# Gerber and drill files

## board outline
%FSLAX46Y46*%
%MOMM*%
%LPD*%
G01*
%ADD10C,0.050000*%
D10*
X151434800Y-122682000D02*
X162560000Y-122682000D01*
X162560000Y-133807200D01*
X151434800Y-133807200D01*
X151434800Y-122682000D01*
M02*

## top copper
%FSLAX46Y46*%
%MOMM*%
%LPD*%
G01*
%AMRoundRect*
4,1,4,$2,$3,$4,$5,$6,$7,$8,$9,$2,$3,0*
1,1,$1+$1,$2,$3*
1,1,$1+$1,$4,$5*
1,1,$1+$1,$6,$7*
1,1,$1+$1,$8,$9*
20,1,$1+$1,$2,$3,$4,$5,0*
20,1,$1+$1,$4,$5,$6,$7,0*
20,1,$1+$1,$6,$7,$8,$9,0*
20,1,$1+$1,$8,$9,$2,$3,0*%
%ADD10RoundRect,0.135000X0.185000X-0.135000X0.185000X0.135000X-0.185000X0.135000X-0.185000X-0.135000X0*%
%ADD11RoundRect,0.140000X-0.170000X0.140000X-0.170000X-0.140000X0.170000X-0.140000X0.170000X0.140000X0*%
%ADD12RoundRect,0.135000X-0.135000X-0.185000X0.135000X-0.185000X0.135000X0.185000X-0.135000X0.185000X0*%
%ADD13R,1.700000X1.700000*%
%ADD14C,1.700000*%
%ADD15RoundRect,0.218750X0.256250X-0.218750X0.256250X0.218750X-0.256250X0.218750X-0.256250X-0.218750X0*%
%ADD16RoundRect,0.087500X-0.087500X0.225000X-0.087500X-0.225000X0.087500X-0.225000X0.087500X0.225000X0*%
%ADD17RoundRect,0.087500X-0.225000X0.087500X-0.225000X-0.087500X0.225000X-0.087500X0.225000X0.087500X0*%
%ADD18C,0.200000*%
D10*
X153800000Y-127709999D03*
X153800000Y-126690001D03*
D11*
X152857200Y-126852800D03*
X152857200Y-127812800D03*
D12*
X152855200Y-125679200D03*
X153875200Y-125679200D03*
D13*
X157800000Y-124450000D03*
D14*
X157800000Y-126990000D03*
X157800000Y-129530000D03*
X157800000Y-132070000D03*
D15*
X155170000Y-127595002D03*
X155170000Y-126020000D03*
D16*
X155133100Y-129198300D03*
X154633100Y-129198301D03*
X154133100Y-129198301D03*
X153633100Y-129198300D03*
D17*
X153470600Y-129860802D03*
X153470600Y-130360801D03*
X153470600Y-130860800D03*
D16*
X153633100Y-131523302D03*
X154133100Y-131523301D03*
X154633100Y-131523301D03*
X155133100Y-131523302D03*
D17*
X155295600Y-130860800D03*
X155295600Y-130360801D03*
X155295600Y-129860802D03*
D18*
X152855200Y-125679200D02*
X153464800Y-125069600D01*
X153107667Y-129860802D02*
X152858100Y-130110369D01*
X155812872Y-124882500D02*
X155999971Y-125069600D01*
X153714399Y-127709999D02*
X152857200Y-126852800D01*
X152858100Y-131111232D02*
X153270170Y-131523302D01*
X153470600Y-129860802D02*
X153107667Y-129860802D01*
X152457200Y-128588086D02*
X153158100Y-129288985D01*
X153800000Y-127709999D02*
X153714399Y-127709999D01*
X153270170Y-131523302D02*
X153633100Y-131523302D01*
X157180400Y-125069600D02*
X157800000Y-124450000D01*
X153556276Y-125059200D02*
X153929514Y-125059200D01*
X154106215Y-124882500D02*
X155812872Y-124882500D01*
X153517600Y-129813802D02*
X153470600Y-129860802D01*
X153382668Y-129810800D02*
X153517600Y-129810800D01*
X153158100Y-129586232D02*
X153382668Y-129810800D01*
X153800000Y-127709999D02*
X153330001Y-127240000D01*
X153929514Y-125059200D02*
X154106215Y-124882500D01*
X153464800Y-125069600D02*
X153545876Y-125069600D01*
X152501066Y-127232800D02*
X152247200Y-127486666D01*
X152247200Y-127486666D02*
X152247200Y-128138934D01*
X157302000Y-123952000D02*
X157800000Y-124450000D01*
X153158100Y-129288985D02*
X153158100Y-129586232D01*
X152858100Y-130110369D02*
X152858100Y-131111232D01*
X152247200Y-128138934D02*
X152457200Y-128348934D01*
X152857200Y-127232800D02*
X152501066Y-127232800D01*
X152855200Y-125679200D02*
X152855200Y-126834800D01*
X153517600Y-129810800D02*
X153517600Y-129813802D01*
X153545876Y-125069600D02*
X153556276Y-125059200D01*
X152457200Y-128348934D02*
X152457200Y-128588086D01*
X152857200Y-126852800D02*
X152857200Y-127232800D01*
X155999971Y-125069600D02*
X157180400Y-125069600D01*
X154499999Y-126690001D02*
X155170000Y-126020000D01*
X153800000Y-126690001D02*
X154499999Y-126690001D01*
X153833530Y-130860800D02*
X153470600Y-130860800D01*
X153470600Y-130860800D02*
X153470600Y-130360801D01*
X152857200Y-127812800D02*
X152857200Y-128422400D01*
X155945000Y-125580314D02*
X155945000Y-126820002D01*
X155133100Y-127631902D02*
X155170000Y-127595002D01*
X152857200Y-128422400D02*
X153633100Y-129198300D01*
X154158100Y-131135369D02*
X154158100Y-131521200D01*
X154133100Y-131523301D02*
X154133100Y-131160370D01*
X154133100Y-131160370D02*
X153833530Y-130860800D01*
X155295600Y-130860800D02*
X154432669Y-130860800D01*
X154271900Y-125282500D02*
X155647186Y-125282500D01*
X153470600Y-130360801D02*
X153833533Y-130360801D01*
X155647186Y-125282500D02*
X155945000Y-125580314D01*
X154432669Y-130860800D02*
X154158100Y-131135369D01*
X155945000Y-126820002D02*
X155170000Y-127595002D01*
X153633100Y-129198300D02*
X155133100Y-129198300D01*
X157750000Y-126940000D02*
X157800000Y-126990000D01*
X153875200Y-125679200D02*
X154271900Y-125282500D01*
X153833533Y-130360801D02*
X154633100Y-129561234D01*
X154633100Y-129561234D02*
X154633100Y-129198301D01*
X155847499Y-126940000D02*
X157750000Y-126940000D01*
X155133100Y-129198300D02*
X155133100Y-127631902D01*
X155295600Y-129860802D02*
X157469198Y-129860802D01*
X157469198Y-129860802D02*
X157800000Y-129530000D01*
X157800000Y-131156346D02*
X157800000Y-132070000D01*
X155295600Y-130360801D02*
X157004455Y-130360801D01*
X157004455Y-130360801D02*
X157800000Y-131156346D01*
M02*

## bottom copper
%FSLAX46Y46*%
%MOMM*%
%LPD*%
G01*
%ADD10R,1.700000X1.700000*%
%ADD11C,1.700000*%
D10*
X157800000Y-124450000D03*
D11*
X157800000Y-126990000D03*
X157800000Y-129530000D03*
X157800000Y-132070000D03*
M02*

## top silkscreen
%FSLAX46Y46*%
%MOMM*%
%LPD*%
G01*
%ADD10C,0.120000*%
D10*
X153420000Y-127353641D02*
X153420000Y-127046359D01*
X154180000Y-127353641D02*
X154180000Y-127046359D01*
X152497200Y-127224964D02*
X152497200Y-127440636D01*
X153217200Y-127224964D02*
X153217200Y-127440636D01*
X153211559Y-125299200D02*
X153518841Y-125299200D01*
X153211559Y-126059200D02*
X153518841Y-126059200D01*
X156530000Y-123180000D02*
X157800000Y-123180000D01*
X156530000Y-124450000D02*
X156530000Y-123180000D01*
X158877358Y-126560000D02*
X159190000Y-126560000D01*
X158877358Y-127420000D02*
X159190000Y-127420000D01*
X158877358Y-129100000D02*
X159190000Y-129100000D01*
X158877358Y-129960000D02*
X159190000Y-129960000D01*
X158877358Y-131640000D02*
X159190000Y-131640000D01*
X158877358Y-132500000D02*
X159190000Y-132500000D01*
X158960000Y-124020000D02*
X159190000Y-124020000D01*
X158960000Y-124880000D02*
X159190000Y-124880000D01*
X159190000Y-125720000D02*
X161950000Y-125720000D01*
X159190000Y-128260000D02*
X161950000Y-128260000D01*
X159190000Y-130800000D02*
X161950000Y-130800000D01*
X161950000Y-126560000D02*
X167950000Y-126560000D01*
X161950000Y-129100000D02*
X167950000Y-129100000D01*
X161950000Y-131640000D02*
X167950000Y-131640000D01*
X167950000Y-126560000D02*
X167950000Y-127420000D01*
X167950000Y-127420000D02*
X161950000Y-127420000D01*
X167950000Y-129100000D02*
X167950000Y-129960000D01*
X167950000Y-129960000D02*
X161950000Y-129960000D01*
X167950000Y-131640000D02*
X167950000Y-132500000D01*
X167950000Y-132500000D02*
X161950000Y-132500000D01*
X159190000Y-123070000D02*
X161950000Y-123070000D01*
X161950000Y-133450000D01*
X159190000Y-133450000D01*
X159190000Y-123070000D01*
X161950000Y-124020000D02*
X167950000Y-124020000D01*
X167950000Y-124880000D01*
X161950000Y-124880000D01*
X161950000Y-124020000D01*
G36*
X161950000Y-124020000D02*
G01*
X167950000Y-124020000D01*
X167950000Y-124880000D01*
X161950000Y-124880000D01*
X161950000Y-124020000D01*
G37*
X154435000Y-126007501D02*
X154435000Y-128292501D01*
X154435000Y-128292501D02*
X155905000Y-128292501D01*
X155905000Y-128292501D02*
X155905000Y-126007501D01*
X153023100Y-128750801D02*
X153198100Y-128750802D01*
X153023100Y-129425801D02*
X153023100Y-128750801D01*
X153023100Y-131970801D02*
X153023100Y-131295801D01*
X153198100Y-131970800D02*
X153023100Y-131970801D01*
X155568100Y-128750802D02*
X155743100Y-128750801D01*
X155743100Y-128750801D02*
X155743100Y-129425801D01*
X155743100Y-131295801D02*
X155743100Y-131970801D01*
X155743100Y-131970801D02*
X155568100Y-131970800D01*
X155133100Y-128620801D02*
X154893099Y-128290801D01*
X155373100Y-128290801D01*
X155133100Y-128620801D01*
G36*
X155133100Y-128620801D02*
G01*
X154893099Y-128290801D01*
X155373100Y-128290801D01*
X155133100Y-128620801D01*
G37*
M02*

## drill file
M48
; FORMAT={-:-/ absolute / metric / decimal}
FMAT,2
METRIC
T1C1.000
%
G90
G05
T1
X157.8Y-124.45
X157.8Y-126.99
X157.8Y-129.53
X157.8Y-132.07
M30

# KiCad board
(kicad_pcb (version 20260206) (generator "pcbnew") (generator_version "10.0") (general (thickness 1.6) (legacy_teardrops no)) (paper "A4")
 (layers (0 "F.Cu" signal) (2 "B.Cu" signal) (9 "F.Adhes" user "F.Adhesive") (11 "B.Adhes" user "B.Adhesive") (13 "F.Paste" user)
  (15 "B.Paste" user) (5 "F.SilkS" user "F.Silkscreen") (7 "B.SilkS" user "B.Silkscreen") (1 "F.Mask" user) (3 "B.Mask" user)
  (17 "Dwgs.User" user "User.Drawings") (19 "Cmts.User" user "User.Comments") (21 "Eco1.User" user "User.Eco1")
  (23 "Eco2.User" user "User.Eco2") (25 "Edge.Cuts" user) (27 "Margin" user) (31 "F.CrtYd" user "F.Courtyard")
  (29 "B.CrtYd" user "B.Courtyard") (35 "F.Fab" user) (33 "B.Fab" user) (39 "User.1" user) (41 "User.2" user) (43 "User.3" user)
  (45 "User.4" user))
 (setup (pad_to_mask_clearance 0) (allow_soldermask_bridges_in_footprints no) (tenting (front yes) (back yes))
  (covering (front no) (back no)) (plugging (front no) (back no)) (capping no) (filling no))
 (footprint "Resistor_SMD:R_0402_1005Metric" (layer "F.Cu") (at 153.8 127.2 90)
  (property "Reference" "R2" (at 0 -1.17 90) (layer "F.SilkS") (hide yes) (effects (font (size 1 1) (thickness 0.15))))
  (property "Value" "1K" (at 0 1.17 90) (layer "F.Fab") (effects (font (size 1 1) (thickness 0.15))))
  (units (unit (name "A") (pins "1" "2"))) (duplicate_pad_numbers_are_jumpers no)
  (fp_line (start -0.153641 -0.38) (end 0.153641 -0.38) (stroke (width 0.12) (type solid)) (layer "F.SilkS"))
  (fp_line (start -0.153641 0.38) (end 0.153641 0.38) (stroke (width 0.12) (type solid)) (layer "F.SilkS"))
  (pad "1" smd roundrect (at -0.509999 0 90) (size 0.54 0.64) (layers "F.Cu" "F.Mask" "F.Paste") (roundrect_rratio 0.25) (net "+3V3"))
  (pad "2" smd roundrect (at 0.509999 0 90) (size 0.54 0.64) (layers "F.Cu" "F.Mask" "F.Paste") (roundrect_rratio 0.25) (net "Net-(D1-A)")))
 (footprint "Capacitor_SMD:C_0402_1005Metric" (layer "F.Cu") (at 152.8572 127.3328 -90)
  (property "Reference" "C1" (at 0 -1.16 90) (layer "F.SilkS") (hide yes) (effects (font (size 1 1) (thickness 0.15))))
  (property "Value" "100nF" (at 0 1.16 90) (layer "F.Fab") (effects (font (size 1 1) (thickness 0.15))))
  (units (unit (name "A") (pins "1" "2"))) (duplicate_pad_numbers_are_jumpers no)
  (fp_line (start -0.107836 0.36) (end 0.107836 0.36) (stroke (width 0.12) (type solid)) (layer "F.SilkS"))
  (fp_line (start -0.107836 -0.36) (end 0.107836 -0.36) (stroke (width 0.12) (type solid)) (layer "F.SilkS"))
  (pad "1" smd roundrect (at -0.48 0 270) (size 0.56 0.62) (layers "F.Cu" "F.Mask" "F.Paste") (roundrect_rratio 0.25) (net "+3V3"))
  (pad "2" smd roundrect (at 0.48 0 270) (size 0.56 0.62) (layers "F.Cu" "F.Mask" "F.Paste") (roundrect_rratio 0.25) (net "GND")))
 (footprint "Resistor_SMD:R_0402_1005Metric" (layer "F.Cu") (at 153.3652 125.6792)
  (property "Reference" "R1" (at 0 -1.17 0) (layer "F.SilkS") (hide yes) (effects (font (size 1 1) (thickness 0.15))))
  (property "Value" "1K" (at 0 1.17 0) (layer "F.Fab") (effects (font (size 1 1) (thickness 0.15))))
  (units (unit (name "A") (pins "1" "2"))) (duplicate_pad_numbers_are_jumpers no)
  (fp_line (start -0.153641 -0.38) (end 0.153641 -0.38) (stroke (width 0.12) (type solid)) (layer "F.SilkS"))
  (fp_line (start -0.153641 0.38) (end 0.153641 0.38) (stroke (width 0.12) (type solid)) (layer "F.SilkS"))
  (pad "1" smd roundrect (at -0.51 0) (size 0.54 0.64) (layers "F.Cu" "F.Mask" "F.Paste") (roundrect_rratio 0.25) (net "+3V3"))
  (pad "2" smd roundrect (at 0.51 0) (size 0.54 0.64) (layers "F.Cu" "F.Mask" "F.Paste") (roundrect_rratio 0.25) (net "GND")))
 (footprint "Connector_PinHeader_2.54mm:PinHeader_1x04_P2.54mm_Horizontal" (layer "F.Cu") (at 157.8 124.45)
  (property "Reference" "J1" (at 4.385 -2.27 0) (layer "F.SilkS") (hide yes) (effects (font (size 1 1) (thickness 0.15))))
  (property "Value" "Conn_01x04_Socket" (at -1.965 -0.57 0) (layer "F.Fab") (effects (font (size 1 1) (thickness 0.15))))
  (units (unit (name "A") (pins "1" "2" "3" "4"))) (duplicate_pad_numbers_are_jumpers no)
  (fp_line (start -1.27 -1.27) (end 0 -1.27) (stroke (width 0.12) (type solid)) (layer "F.SilkS"))
  (fp_line (start -1.27 0) (end -1.27 -1.27) (stroke (width 0.12) (type solid)) (layer "F.SilkS"))
  (fp_line (start 1.077358 2.11) (end 1.39 2.11) (stroke (width 0.12) (type solid)) (layer "F.SilkS"))
  (fp_line (start 1.077358 2.97) (end 1.39 2.97) (stroke (width 0.12) (type solid)) (layer "F.SilkS"))
  (fp_line (start 1.077358 4.65) (end 1.39 4.65) (stroke (width 0.12) (type solid)) (layer "F.SilkS"))
  (fp_line (start 1.077358 5.51) (end 1.39 5.51) (stroke (width 0.12) (type solid)) (layer "F.SilkS"))
  (fp_line (start 1.077358 7.19) (end 1.39 7.19) (stroke (width 0.12) (type solid)) (layer "F.SilkS"))
  (fp_line (start 1.077358 8.05) (end 1.39 8.05) (stroke (width 0.12) (type solid)) (layer "F.SilkS"))
  (fp_line (start 1.16 -0.43) (end 1.39 -0.43) (stroke (width 0.12) (type solid)) (layer "F.SilkS"))
  (fp_line (start 1.16 0.43) (end 1.39 0.43) (stroke (width 0.12) (type solid)) (layer "F.SilkS"))
  (fp_line (start 1.39 1.27) (end 4.15 1.27) (stroke (width 0.12) (type solid)) (layer "F.SilkS"))
  (fp_line (start 1.39 3.81) (end 4.15 3.81) (stroke (width 0.12) (type solid)) (layer "F.SilkS"))
  (fp_line (start 1.39 6.35) (end 4.15 6.35) (stroke (width 0.12) (type solid)) (layer "F.SilkS"))
  (fp_line (start 4.15 2.11) (end 10.15 2.11) (stroke (width 0.12) (type solid)) (layer "F.SilkS"))
  (fp_line (start 4.15 4.65) (end 10.15 4.65) (stroke (width 0.12) (type solid)) (layer "F.SilkS"))
  (fp_line (start 4.15 7.19) (end 10.15 7.19) (stroke (width 0.12) (type solid)) (layer "F.SilkS"))
  (fp_line (start 10.15 2.11) (end 10.15 2.97) (stroke (width 0.12) (type solid)) (layer "F.SilkS"))
  (fp_line (start 10.15 2.97) (end 4.15 2.97) (stroke (width 0.12) (type solid)) (layer "F.SilkS"))
  (fp_line (start 10.15 4.65) (end 10.15 5.51) (stroke (width 0.12) (type solid)) (layer "F.SilkS"))
  (fp_line (start 10.15 5.51) (end 4.15 5.51) (stroke (width 0.12) (type solid)) (layer "F.SilkS"))
  (fp_line (start 10.15 7.19) (end 10.15 8.05) (stroke (width 0.12) (type solid)) (layer "F.SilkS"))
  (fp_line (start 10.15 8.05) (end 4.15 8.05) (stroke (width 0.12) (type solid)) (layer "F.SilkS"))
  (fp_rect (start 1.39 -1.38) (end 4.15 9) (stroke (width 0.12) (type solid)) (fill no) (layer "F.SilkS"))
  (fp_rect (start 4.15 -0.43) (end 10.15 0.43) (stroke (width 0.12) (type solid)) (fill yes) (layer "F.SilkS"))
  (pad "1" thru_hole rect (at 0 0) (size 1.7 1.7) (drill 1) (layers "*.Cu" "*.Mask") (remove_unused_layers no) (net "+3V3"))
  (pad "2" thru_hole circle (at 0 2.54) (size 1.7 1.7) (drill 1) (layers "*.Cu" "*.Mask") (remove_unused_layers no) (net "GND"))
  (pad "3" thru_hole circle (at 0 5.08) (size 1.7 1.7) (drill 1) (layers "*.Cu" "*.Mask") (remove_unused_layers no) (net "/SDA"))
  (pad "4" thru_hole circle (at 0 7.62) (size 1.7 1.7) (drill 1) (layers "*.Cu" "*.Mask") (remove_unused_layers no) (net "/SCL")))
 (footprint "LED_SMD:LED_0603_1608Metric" (layer "F.Cu") (at 155.17 126.807501 90)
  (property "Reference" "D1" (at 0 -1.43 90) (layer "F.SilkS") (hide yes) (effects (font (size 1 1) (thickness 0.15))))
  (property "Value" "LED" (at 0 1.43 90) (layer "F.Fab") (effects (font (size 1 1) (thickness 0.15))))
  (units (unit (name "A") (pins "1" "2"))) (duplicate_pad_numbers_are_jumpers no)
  (fp_line (start 0.8 -0.735) (end -1.485 -0.735) (stroke (width 0.12) (type solid)) (layer "F.SilkS"))
  (fp_line (start -1.485 -0.735) (end -1.485 0.735) (stroke (width 0.12) (type solid)) (layer "F.SilkS"))
  (fp_line (start -1.485 0.735) (end 0.8 0.735) (stroke (width 0.12) (type solid)) (layer "F.SilkS"))
  (pad "1" smd roundrect (at -0.787501 0 90) (size 0.875 0.95) (layers "F.Cu" "F.Mask" "F.Paste") (roundrect_rratio 0.25) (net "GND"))
  (pad "2" smd roundrect (at 0.787501 0 90) (size 0.875 0.95) (layers "F.Cu" "F.Mask" "F.Paste") (roundrect_rratio 0.25) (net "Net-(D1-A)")))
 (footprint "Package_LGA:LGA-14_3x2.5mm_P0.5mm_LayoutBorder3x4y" (layer "F.Cu") (at 154.3831 130.360801 -90)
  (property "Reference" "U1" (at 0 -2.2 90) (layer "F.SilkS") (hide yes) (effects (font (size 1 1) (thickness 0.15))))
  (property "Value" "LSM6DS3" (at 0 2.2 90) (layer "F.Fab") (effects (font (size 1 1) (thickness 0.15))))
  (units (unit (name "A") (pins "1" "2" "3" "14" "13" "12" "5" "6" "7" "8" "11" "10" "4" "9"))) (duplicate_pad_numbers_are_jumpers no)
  (fp_line (start -1.61 1.36) (end -1.609999 1.185) (stroke (width 0.12) (type solid)) (layer "F.SilkS"))
  (fp_line (start -0.935 1.36) (end -1.61 1.36) (stroke (width 0.12) (type solid)) (layer "F.SilkS"))
  (fp_line (start 1.61 1.36) (end 0.935 1.36) (stroke (width 0.12) (type solid)) (layer "F.SilkS"))
  (fp_line (start 1.609999 1.185) (end 1.61 1.36) (stroke (width 0.12) (type solid)) (layer "F.SilkS"))
  (fp_line (start -1.609999 -1.185) (end -1.61 -1.36) (stroke (width 0.12) (type solid)) (layer "F.SilkS"))
  (fp_line (start -1.61 -1.36) (end -0.935 -1.36) (stroke (width 0.12) (type solid)) (layer "F.SilkS"))
  (fp_line (start 0.935 -1.36) (end 1.61 -1.36) (stroke (width 0.12) (type solid)) (layer "F.SilkS"))
  (fp_line (start 1.61 -1.36) (end 1.609999 -1.185) (stroke (width 0.12) (type solid)) (layer "F.SilkS"))
  (fp_poly (pts (xy -1.74 -0.75) (xy -2.07 -0.509999) (xy -2.07 -0.99)) (stroke (width 0.12) (type solid)) (fill yes) (layer "F.SilkS"))
  (pad "1" smd roundrect (at -1.162501 -0.75 270) (size 0.625 0.35) (layers "F.Cu" "F.Mask" "F.Paste") (roundrect_rratio 0.25) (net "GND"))
  (pad "2" smd roundrect (at -1.1625 -0.25 270) (size 0.625 0.35) (layers "F.Cu" "F.Mask" "F.Paste") (roundrect_rratio 0.25) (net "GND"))
  (pad "3" smd roundrect (at -1.1625 0.25 270) (size 0.625 0.35) (layers "F.Cu" "F.Mask" "F.Paste") (roundrect_rratio 0.25) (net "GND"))
  (pad "4" smd roundrect (at -1.162501 0.75 270) (size 0.625 0.35) (layers "F.Cu" "F.Mask" "F.Paste") (roundrect_rratio 0.25) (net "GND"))
  (pad "5" smd roundrect (at -0.499999 0.9125 270) (size 0.35 0.625) (layers "F.Cu" "F.Mask" "F.Paste") (roundrect_rratio 0.25) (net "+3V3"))
  (pad "6" smd roundrect (at 0 0.9125 270) (size 0.35 0.625) (layers "F.Cu" "F.Mask" "F.Paste") (roundrect_rratio 0.25) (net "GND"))
  (pad "7" smd roundrect (at 0.499999 0.9125 270) (size 0.35 0.625) (layers "F.Cu" "F.Mask" "F.Paste") (roundrect_rratio 0.25) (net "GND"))
  (pad "8" smd roundrect (at 1.162501 0.75 270) (size 0.625 0.35) (layers "F.Cu" "F.Mask" "F.Paste") (roundrect_rratio 0.25) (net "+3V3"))
  (pad "9" smd roundrect (at 1.1625 0.25 270) (size 0.625 0.35) (layers "F.Cu" "F.Mask" "F.Paste") (roundrect_rratio 0.25) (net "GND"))
  (pad "10" smd roundrect (at 1.1625 -0.25 270) (size 0.625 0.35) (layers "F.Cu" "F.Mask" "F.Paste") (roundrect_rratio 0.25)
   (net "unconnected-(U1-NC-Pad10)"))
  (pad "11" smd roundrect (at 1.162501 -0.75 270) (size 0.625 0.35) (layers "F.Cu" "F.Mask" "F.Paste") (roundrect_rratio 0.25)
   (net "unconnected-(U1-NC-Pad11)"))
  (pad "12" smd roundrect (at 0.499999 -0.9125 270) (size 0.35 0.625) (layers "F.Cu" "F.Mask" "F.Paste") (roundrect_rratio 0.25) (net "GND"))
  (pad "13" smd roundrect (at 0 -0.9125 270) (size 0.35 0.625) (layers "F.Cu" "F.Mask" "F.Paste") (roundrect_rratio 0.25) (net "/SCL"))
  (pad "14" smd roundrect (at -0.499999 -0.9125 270) (size 0.35 0.625) (layers "F.Cu" "F.Mask" "F.Paste") (roundrect_rratio 0.25)
   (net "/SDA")))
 (gr_rect (start 151.4348 122.682) (end 162.56 133.8072) (stroke (width 0.05) (type default)) (fill no) (layer "Edge.Cuts"))
 (segment (start 152.8552 125.6792) (end 153.4648 125.0696) (width 0.2) (layer "F.Cu") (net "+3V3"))
 (segment (start 153.107667 129.860802) (end 152.8581 130.110369) (width 0.2) (layer "F.Cu") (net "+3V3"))
 (segment (start 155.812872 124.8825) (end 155.999971 125.0696) (width 0.2) (layer "F.Cu") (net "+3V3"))
 (segment (start 153.714399 127.709999) (end 152.8572 126.8528) (width 0.2) (layer "F.Cu") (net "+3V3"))
 (segment (start 152.8581 131.111232) (end 153.27017 131.523302) (width 0.2) (layer "F.Cu") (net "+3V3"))
 (segment (start 153.4706 129.860802) (end 153.107667 129.860802) (width 0.2) (layer "F.Cu") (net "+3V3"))
 (segment (start 152.4572 128.588086) (end 153.1581 129.288985) (width 0.2) (layer "F.Cu") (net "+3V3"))
 (segment (start 153.8 127.709999) (end 153.714399 127.709999) (width 0.2) (layer "F.Cu") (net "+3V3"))
 (segment (start 153.27017 131.523302) (end 153.6331 131.523302) (width 0.2) (layer "F.Cu") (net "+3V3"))
 (segment (start 157.1804 125.0696) (end 157.8 124.45) (width 0.2) (layer "F.Cu") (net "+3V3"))
 (segment (start 153.556276 125.0592) (end 153.929514 125.0592) (width 0.2) (layer "F.Cu") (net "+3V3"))
 (segment (start 154.106215 124.8825) (end 155.812872 124.8825) (width 0.2) (layer "F.Cu") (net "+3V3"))
 (segment (start 153.5176 129.813802) (end 153.4706 129.860802) (width 0.2) (layer "F.Cu") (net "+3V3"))
 (segment (start 153.382668 129.8108) (end 153.5176 129.8108) (width 0.2) (layer "F.Cu") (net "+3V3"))
 (segment (start 153.1581 129.586232) (end 153.382668 129.8108) (width 0.2) (layer "F.Cu") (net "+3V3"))
 (segment (start 153.8 127.709999) (end 153.330001 127.24) (width 0.2) (layer "F.Cu") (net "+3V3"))
 (segment (start 153.929514 125.0592) (end 154.106215 124.8825) (width 0.2) (layer "F.Cu") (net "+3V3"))
 (segment (start 153.4648 125.0696) (end 153.545876 125.0696) (width 0.2) (layer "F.Cu") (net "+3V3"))
 (segment (start 152.501066 127.2328) (end 152.2472 127.486666) (width 0.2) (layer "F.Cu") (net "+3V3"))
 (segment (start 152.2472 127.486666) (end 152.2472 128.138934) (width 0.2) (layer "F.Cu") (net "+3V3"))
 (segment (start 157.302 123.952) (end 157.8 124.45) (width 0.2) (layer "F.Cu") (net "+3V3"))
 (segment (start 153.1581 129.288985) (end 153.1581 129.586232) (width 0.2) (layer "F.Cu") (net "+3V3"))
 (segment (start 152.8581 130.110369) (end 152.8581 131.111232) (width 0.2) (layer "F.Cu") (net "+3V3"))
 (segment (start 152.2472 128.138934) (end 152.4572 128.348934) (width 0.2) (layer "F.Cu") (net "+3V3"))
 (segment (start 152.8572 127.2328) (end 152.501066 127.2328) (width 0.2) (layer "F.Cu") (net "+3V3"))
 (segment (start 152.8552 125.6792) (end 152.8552 126.8348) (width 0.2) (layer "F.Cu") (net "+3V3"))
 (segment (start 153.5176 129.8108) (end 153.5176 129.813802) (width 0.2) (layer "F.Cu") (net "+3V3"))
 (segment (start 153.545876 125.0696) (end 153.556276 125.0592) (width 0.2) (layer "F.Cu") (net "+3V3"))
 (segment (start 152.4572 128.348934) (end 152.4572 128.588086) (width 0.2) (layer "F.Cu") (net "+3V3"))
 (segment (start 152.8572 126.8528) (end 152.8572 127.2328) (width 0.2) (layer "F.Cu") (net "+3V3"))
 (segment (start 155.999971 125.0696) (end 157.1804 125.0696) (width 0.2) (layer "F.Cu") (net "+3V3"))
 (segment (start 154.499999 126.690001) (end 155.17 126.02) (width 0.2) (layer "F.Cu") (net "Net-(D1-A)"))
 (segment (start 153.8 126.690001) (end 154.499999 126.690001) (width 0.2) (layer "F.Cu") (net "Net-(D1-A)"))
 (segment (start 153.83353 130.8608) (end 153.4706 130.8608) (width 0.2) (layer "F.Cu") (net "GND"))
 (segment (start 153.4706 130.8608) (end 153.4706 130.360801) (width 0.2) (layer "F.Cu") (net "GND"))
 (segment (start 152.8572 127.8128) (end 152.8572 128.4224) (width 0.2) (layer "F.Cu") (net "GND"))
 (segment (start 155.945 125.580314) (end 155.945 126.820002) (width 0.2) (layer "F.Cu") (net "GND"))
 (segment (start 155.1331 127.631902) (end 155.17 127.595002) (width 0.2) (layer "F.Cu") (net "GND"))
 (segment (start 152.8572 128.4224) (end 153.6331 129.1983) (width 0.2) (layer "F.Cu") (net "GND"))
 (segment (start 154.1581 131.135369) (end 154.1581 131.5212) (width 0.2) (layer "F.Cu") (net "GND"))
 (segment (start 154.1331 131.523301) (end 154.1331 131.16037) (width 0.2) (layer "F.Cu") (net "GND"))
 (segment (start 154.1331 131.16037) (end 153.83353 130.8608) (width 0.2) (layer "F.Cu") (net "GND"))
 (segment (start 155.2956 130.8608) (end 154.432669 130.8608) (width 0.2) (layer "F.Cu") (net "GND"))
 (segment (start 154.2719 125.2825) (end 155.647186 125.2825) (width 0.2) (layer "F.Cu") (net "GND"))
 (segment (start 153.4706 130.360801) (end 153.833533 130.360801) (width 0.2) (layer "F.Cu") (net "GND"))
 (segment (start 155.647186 125.2825) (end 155.945 125.580314) (width 0.2) (layer "F.Cu") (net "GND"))
 (segment (start 154.432669 130.8608) (end 154.1581 131.135369) (width 0.2) (layer "F.Cu") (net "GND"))
 (segment (start 155.945 126.820002) (end 155.17 127.595002) (width 0.2) (layer "F.Cu") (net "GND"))
 (segment (start 153.6331 129.1983) (end 155.1331 129.1983) (width 0.2) (layer "F.Cu") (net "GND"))
 (segment (start 157.75 126.94) (end 157.8 126.99) (width 0.2) (layer "F.Cu") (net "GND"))
 (segment (start 153.8752 125.6792) (end 154.2719 125.2825) (width 0.2) (layer "F.Cu") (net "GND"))
 (segment (start 153.833533 130.360801) (end 154.6331 129.561234) (width 0.2) (layer "F.Cu") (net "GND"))
 (segment (start 154.6331 129.561234) (end 154.6331 129.198301) (width 0.2) (layer "F.Cu") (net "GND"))
 (segment (start 155.847499 126.94) (end 157.75 126.94) (width 0.2) (layer "F.Cu") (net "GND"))
 (segment (start 155.1331 129.1983) (end 155.1331 127.631902) (width 0.2) (layer "F.Cu") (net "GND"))
 (segment (start 155.2956 129.860802) (end 157.469198 129.860802) (width 0.2) (layer "F.Cu") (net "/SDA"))
 (segment (start 157.469198 129.860802) (end 157.8 129.53) (width 0.2) (layer "F.Cu") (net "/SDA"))
 (segment (start 157.8 131.156346) (end 157.8 132.07) (width 0.2) (layer "F.Cu") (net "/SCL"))
 (segment (start 155.2956 130.360801) (end 157.004455 130.360801) (width 0.2) (layer "F.Cu") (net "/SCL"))
 (segment (start 157.004455 130.360801) (end 157.8 131.156346) (width 0.2) (layer "F.Cu") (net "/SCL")))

